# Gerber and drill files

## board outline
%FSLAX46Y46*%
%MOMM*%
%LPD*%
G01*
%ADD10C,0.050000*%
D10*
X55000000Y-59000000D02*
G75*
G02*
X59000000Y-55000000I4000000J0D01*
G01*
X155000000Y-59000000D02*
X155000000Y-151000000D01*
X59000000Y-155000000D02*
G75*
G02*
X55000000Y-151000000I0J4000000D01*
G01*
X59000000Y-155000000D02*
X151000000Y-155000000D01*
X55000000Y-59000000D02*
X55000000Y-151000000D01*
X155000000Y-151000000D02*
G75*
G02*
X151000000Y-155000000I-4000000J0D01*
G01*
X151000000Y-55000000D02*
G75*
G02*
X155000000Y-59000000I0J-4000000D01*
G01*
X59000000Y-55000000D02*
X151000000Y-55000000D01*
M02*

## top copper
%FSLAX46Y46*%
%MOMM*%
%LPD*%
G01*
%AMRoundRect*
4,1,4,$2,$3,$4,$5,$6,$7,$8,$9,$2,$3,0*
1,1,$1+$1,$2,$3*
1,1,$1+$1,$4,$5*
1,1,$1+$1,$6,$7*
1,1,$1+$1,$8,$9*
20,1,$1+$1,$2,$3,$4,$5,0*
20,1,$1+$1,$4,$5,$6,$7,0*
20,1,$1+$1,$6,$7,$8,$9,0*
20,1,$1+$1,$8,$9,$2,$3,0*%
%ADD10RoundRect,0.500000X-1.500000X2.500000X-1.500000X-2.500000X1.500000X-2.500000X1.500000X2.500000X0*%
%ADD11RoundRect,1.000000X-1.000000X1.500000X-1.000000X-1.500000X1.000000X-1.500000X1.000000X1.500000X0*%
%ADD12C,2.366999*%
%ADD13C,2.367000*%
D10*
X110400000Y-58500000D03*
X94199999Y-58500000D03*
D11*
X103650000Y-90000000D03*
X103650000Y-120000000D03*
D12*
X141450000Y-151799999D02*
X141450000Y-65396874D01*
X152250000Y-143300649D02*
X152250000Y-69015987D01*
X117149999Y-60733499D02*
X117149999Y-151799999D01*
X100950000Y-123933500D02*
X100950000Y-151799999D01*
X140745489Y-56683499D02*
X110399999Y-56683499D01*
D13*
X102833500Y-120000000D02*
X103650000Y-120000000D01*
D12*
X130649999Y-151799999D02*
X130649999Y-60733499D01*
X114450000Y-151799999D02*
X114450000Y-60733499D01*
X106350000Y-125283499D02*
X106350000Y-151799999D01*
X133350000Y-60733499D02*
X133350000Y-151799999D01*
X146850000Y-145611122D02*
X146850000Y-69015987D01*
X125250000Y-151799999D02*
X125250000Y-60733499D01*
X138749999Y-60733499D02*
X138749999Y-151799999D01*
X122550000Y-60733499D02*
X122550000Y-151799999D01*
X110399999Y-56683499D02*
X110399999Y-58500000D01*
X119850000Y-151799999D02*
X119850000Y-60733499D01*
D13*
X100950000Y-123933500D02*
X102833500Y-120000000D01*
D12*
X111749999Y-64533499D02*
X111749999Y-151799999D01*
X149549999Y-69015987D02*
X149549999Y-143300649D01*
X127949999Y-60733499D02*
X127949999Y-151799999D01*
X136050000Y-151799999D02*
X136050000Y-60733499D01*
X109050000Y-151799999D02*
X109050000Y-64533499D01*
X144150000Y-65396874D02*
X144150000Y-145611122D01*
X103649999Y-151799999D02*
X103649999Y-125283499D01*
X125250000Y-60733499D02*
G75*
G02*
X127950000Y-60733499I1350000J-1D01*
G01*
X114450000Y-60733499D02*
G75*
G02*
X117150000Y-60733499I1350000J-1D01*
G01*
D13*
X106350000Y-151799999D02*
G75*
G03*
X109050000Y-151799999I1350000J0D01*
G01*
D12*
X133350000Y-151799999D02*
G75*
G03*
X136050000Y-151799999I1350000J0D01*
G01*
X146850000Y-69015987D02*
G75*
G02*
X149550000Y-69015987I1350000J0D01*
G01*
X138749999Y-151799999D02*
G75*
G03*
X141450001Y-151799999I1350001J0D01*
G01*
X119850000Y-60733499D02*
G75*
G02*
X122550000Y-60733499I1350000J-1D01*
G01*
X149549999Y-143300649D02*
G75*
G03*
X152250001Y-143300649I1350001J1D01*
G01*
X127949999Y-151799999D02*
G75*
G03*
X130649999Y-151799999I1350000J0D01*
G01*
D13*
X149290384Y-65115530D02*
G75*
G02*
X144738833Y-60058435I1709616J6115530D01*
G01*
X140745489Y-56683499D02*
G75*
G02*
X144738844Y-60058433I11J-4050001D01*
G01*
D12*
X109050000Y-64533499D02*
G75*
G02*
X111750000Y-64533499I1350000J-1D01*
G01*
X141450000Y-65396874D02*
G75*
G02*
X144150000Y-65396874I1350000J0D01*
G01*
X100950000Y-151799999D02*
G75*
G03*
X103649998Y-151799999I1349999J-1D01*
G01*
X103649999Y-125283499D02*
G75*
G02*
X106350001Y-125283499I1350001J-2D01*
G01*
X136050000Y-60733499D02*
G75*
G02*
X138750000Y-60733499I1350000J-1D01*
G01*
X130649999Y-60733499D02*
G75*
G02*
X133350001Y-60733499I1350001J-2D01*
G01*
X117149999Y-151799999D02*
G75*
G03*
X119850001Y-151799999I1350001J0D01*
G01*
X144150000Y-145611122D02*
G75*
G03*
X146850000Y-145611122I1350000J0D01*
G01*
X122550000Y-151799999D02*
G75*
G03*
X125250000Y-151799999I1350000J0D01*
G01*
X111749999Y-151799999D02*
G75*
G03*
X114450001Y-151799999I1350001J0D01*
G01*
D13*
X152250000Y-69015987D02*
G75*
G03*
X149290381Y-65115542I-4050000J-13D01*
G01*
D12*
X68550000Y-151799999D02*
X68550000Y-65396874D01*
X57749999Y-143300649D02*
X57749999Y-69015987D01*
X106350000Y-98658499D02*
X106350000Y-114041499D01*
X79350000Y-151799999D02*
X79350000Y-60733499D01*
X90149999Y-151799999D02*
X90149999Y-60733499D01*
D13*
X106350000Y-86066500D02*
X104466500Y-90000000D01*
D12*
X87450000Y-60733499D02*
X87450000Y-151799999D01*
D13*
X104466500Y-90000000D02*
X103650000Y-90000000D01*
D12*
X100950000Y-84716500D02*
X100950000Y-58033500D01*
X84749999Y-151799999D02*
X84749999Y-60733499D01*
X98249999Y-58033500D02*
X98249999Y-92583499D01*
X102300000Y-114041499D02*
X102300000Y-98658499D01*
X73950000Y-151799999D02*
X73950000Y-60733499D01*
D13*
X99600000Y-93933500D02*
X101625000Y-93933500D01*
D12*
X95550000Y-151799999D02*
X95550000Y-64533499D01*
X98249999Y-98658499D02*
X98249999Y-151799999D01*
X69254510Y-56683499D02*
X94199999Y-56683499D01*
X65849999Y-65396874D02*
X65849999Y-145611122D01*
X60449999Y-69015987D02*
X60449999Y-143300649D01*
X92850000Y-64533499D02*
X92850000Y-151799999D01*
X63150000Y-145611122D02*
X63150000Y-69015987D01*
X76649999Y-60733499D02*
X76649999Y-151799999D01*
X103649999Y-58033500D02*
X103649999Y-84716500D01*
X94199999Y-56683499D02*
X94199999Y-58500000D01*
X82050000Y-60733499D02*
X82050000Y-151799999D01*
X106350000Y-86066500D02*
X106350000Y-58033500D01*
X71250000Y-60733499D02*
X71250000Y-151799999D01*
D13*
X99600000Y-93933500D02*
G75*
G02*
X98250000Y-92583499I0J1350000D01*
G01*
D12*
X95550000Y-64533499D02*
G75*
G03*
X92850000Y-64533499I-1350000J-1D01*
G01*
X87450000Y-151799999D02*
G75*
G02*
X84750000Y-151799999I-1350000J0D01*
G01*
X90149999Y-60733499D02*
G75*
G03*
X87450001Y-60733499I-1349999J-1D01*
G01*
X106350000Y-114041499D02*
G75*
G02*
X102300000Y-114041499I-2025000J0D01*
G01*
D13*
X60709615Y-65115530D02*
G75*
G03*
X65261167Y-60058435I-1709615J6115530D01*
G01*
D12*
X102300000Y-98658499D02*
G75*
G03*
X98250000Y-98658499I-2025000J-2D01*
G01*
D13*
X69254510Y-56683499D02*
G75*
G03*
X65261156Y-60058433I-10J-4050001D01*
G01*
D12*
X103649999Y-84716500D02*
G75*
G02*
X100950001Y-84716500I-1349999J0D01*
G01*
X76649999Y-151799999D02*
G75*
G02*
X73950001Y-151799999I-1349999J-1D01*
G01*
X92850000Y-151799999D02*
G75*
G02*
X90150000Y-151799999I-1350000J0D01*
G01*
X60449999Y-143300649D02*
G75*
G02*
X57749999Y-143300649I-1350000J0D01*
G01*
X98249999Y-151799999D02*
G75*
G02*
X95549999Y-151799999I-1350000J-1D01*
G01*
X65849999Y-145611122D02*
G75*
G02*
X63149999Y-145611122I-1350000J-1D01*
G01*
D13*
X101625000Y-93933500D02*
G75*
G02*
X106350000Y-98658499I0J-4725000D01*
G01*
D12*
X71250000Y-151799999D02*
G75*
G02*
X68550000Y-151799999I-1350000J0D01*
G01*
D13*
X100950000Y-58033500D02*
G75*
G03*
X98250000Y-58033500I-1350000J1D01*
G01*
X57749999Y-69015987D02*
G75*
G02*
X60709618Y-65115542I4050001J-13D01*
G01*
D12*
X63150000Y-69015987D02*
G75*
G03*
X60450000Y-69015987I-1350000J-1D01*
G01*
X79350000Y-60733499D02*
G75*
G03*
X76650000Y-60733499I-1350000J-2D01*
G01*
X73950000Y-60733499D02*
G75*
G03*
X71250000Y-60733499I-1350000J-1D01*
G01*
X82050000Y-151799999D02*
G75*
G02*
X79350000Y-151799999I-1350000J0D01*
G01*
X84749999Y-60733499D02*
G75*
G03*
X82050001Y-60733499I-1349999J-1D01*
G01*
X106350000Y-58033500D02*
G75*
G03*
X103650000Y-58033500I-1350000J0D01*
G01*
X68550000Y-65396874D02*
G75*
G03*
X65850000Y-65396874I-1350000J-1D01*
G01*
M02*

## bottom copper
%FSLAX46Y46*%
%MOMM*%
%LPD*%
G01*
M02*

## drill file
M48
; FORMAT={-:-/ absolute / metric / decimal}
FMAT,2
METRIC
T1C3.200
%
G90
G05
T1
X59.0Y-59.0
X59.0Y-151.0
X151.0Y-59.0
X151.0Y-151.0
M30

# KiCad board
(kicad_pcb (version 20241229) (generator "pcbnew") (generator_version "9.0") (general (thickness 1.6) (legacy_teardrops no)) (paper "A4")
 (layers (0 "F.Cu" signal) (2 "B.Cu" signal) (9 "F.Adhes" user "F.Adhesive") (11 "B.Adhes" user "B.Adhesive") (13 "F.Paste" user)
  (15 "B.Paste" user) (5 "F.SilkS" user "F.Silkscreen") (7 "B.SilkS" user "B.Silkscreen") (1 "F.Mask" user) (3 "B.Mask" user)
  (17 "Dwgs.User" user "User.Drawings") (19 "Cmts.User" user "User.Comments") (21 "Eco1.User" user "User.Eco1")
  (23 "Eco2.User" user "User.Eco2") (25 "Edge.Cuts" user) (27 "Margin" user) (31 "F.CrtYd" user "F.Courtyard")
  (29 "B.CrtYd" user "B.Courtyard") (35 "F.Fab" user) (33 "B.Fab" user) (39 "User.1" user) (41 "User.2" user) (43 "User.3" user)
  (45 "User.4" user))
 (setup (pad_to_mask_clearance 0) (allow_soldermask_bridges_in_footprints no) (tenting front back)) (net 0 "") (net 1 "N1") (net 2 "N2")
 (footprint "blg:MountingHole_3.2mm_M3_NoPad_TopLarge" (layer "F.Cu") (at 151 59)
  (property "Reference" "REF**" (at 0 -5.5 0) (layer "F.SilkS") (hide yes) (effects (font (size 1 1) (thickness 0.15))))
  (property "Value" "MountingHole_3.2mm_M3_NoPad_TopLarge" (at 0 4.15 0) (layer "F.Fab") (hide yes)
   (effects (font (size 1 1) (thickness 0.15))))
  (pad "" np_thru_hole circle (at 0 0) (size 7.6 7.6) (drill 3.2) (layers) (zone_connect 2)))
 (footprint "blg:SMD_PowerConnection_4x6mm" (layer "F.Cu") (at 110.4 58.5 -90)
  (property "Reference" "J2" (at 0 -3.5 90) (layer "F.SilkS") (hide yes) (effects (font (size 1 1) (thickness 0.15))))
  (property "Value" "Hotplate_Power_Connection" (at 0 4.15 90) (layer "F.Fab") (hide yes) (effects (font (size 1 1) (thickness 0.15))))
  (pad "1" smd roundrect (at 0 0 270) (size 6 4) (layers "F.Cu" "F.Mask" "F.Paste") (roundrect_rratio 0.125) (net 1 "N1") (zone_connect 2)))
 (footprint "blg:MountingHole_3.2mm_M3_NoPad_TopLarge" (layer "F.Cu") (at 59 151)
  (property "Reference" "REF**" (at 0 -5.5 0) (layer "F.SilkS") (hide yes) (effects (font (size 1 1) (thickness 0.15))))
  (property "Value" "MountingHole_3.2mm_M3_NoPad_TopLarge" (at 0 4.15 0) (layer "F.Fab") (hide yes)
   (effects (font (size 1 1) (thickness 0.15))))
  (pad "" np_thru_hole circle (at 0 0) (size 7.6 7.6) (drill 3.2) (layers) (zone_connect 2)))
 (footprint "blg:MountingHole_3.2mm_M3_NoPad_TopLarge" (layer "F.Cu") (at 151 151)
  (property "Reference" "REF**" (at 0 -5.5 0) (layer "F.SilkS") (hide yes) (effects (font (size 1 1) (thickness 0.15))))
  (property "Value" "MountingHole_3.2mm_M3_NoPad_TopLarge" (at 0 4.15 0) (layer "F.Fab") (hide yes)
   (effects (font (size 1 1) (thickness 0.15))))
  (pad "" np_thru_hole circle (at 0 0) (size 7.6 7.6) (drill 3.2) (layers) (zone_connect 2)))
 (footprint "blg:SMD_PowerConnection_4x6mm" (layer "F.Cu") (at 94.199999 58.5 -90)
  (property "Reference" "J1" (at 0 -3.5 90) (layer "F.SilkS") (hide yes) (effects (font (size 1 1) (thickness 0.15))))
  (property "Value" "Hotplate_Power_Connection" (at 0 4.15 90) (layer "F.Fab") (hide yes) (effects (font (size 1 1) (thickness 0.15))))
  (pad "1" smd roundrect (at 0 0 270) (size 6 4) (layers "F.Cu" "F.Mask" "F.Paste") (roundrect_rratio 0.125) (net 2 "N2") (zone_connect 2)))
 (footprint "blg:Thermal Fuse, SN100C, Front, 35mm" (layer "F.Cu") (at 103.65 105 -90)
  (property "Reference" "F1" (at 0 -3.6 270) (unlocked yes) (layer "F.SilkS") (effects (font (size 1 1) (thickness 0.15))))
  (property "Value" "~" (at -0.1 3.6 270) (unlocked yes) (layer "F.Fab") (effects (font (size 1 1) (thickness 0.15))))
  (pad "1" smd roundrect (at -15 0 270) (size 5 4) (layers "F.Cu" "F.Mask") (roundrect_rratio 0.25) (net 2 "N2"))
  (pad "2" smd roundrect (at 15 0 270) (size 5 4) (layers "F.Cu" "F.Mask") (roundrect_rratio 0.25) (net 1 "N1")))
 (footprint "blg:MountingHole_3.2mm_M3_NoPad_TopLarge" (layer "F.Cu") (at 59 59)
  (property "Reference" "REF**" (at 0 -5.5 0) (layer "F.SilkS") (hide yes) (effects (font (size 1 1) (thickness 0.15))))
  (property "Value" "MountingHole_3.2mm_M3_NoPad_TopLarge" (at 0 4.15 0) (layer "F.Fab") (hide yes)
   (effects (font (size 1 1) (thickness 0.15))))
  (pad "" np_thru_hole circle (at 0 0) (size 7.6 7.6) (drill 3.2) (layers) (zone_connect 2)))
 (gr_arc (start 55 59) (mid 56.171573 56.171573) (end 59 55) (stroke (width 0.05) (type solid)) (layer "Edge.Cuts"))
 (gr_line (start 155 59) (end 155 151) (stroke (width 0.05) (type default)) (layer "Edge.Cuts"))
 (gr_arc (start 59 155) (mid 56.171573 153.828427) (end 55 151) (stroke (width 0.05) (type solid)) (layer "Edge.Cuts"))
 (gr_line (start 59 155) (end 151 155) (stroke (width 0.05) (type default)) (layer "Edge.Cuts"))
 (gr_line (start 55 59) (end 55 151) (stroke (width 0.05) (type default)) (layer "Edge.Cuts"))
 (gr_arc (start 155 151) (mid 153.828427 153.828427) (end 151 155) (stroke (width 0.05) (type solid)) (layer "Edge.Cuts"))
 (gr_arc (start 151 55) (mid 153.828427 56.171573) (end 155 59) (stroke (width 0.05) (type solid)) (layer "Edge.Cuts"))
 (gr_line (start 59 55) (end 151 55) (stroke (width 0.05) (type default)) (layer "Edge.Cuts"))
 (segment (start 141.45 151.799999) (end 141.45 65.396874) (width 2.366999) (layer "F.Cu") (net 1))
 (segment (start 152.25 143.300649) (end 152.25 69.015987) (width 2.366999) (layer "F.Cu") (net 1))
 (segment (start 117.149999 60.733499) (end 117.149999 151.799999) (width 2.366999) (layer "F.Cu") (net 1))
 (segment (start 100.95 123.9335) (end 100.95 151.799999) (width 2.366999) (layer "F.Cu") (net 1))
 (segment (start 140.745489 56.683499) (end 110.399999 56.683499) (width 2.366999) (layer "F.Cu") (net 1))
 (segment (start 102.8335 120) (end 103.65 120) (width 2.367) (layer "F.Cu") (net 1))
 (segment (start 130.649999 151.799999) (end 130.649999 60.733499) (width 2.366999) (layer "F.Cu") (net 1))
 (segment (start 114.45 151.799999) (end 114.45 60.733499) (width 2.366999) (layer "F.Cu") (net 1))
 (segment (start 106.35 125.283499) (end 106.35 151.799999) (width 2.366999) (layer "F.Cu") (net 1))
 (segment (start 133.35 60.733499) (end 133.35 151.799999) (width 2.366999) (layer "F.Cu") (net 1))
 (segment (start 146.85 145.611122) (end 146.85 69.015987) (width 2.366999) (layer "F.Cu") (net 1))
 (segment (start 125.25 151.799999) (end 125.25 60.733499) (width 2.366999) (layer "F.Cu") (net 1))
 (segment (start 138.749999 60.733499) (end 138.749999 151.799999) (width 2.366999) (layer "F.Cu") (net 1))
 (segment (start 122.55 60.733499) (end 122.55 151.799999) (width 2.366999) (layer "F.Cu") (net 1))
 (segment (start 110.399999 56.683499) (end 110.399999 58.5) (width 2.366999) (layer "F.Cu") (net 1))
 (segment (start 119.85 151.799999) (end 119.85 60.733499) (width 2.366999) (layer "F.Cu") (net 1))
 (segment (start 100.95 123.9335) (end 102.8335 120) (width 2.367) (layer "F.Cu") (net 1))
 (segment (start 111.749999 64.533499) (end 111.749999 151.799999) (width 2.366999) (layer "F.Cu") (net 1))
 (segment (start 149.549999 69.015987) (end 149.549999 143.300649) (width 2.366999) (layer "F.Cu") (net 1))
 (segment (start 127.949999 60.733499) (end 127.949999 151.799999) (width 2.366999) (layer "F.Cu") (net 1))
 (segment (start 136.05 151.799999) (end 136.05 60.733499) (width 2.366999) (layer "F.Cu") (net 1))
 (segment (start 109.05 151.799999) (end 109.05 64.533499) (width 2.366999) (layer "F.Cu") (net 1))
 (segment (start 144.15 65.396874) (end 144.15 145.611122) (width 2.366999) (layer "F.Cu") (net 1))
 (segment (start 103.649999 151.799999) (end 103.649999 125.283499) (width 2.366999) (layer "F.Cu") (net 1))
 (arc (start 125.25 60.733499) (mid 126.6 59.3835) (end 127.949999 60.733499) (width 2.366999) (layer "F.Cu") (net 1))
 (arc (start 114.45 60.733499) (mid 115.8 59.3835) (end 117.149999 60.733499) (width 2.366999) (layer "F.Cu") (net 1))
 (arc (start 106.35 151.799999) (mid 107.7 153.149999) (end 109.05 151.799999) (width 2.367) (layer "F.Cu") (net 1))
 (arc (start 133.35 151.799999) (mid 134.7 153.149999) (end 136.05 151.799999) (width 2.366999) (layer "F.Cu") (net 1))
 (arc (start 146.85 69.015987) (mid 148.2 67.665987) (end 149.549999 69.015987) (width 2.366999) (layer "F.Cu") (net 1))
 (arc (start 138.749999 151.799999) (mid 140.1 153.149999) (end 141.45 151.799999) (width 2.366999) (layer "F.Cu") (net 1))
 (arc (start 119.85 60.733499) (mid 121.199999 59.3835) (end 122.55 60.733499) (width 2.366999) (layer "F.Cu") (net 1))
 (arc (start 149.549999 143.300649) (mid 150.9 144.650649) (end 152.25 143.300649) (width 2.366999) (layer "F.Cu") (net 1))
 (arc (start 127.949999 151.799999) (mid 129.3 153.149999) (end 130.649999 151.799999) (width 2.366999) (layer "F.Cu") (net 1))
 (arc (start 149.290384 65.11553) (mid 146.280159 63.248011) (end 144.738832 60.058435) (width 2.367) (layer "F.Cu") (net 1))
 (arc (start 140.745489 56.683499) (mid 143.359728 57.64024) (end 144.738832 60.058435) (width 2.367) (layer "F.Cu") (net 1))
 (arc (start 109.05 64.533499) (mid 110.399999 63.1835) (end 111.749999 64.533499) (width 2.366999) (layer "F.Cu") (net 1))
 (arc (start 141.45 65.396874) (mid 142.799999 64.046874) (end 144.15 65.396874) (width 2.366999) (layer "F.Cu") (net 1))
 (arc (start 100.95 151.799999) (mid 102.3 153.149999) (end 103.649999 151.799999) (width 2.366999) (layer "F.Cu") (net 1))
 (arc (start 103.649999 125.283499) (mid 105 123.9335) (end 106.35 125.283499) (width 2.366999) (layer "F.Cu") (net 1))
 (arc (start 136.05 60.733499) (mid 137.4 59.3835) (end 138.749999 60.733499) (width 2.366999) (layer "F.Cu") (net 1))
 (arc (start 130.649999 60.733499) (mid 132 59.3835) (end 133.35 60.733499) (width 2.366999) (layer "F.Cu") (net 1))
 (arc (start 117.149999 151.799999) (mid 118.5 153.149999) (end 119.85 151.799999) (width 2.366999) (layer "F.Cu") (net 1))
 (arc (start 144.15 145.611122) (mid 145.5 146.961122) (end 146.85 145.611122) (width 2.366999) (layer "F.Cu") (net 1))
 (arc (start 122.55 151.799999) (mid 123.899999 153.149999) (end 125.25 151.799999) (width 2.366999) (layer "F.Cu") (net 1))
 (arc (start 111.749999 151.799999) (mid 113.1 153.149999) (end 114.45 151.799999) (width 2.366999) (layer "F.Cu") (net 1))
 (arc (start 152.25 69.015987) (mid 151.04468 66.133229) (end 149.290384 65.11553) (width 2.367) (layer "F.Cu") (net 1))
 (segment (start 68.55 151.799999) (end 68.55 65.396874) (width 2.366999) (layer "F.Cu") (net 2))
 (segment (start 57.749999 143.300649) (end 57.749999 69.015987) (width 2.366999) (layer "F.Cu") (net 2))
 (segment (start 106.35 98.658499) (end 106.35 114.041499) (width 2.366999) (layer "F.Cu") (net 2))
 (segment (start 79.35 151.799999) (end 79.35 60.733499) (width 2.366999) (layer "F.Cu") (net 2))
 (segment (start 90.149999 151.799999) (end 90.149999 60.733499) (width 2.366999) (layer "F.Cu") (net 2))
 (segment (start 106.35 86.0665) (end 104.4665 90) (width 2.367) (layer "F.Cu") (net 2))
 (segment (start 87.45 60.733499) (end 87.45 151.799999) (width 2.366999) (layer "F.Cu") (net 2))
 (segment (start 104.4665 90) (end 103.65 90) (width 2.367) (layer "F.Cu") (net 2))
 (segment (start 100.95 84.7165) (end 100.95 58.0335) (width 2.366999) (layer "F.Cu") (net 2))
 (segment (start 84.749999 151.799999) (end 84.749999 60.733499) (width 2.366999) (layer "F.Cu") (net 2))
 (segment (start 98.249999 58.0335) (end 98.249999 92.583499) (width 2.366999) (layer "F.Cu") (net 2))
 (segment (start 102.3 114.041499) (end 102.3 98.658499) (width 2.366999) (layer "F.Cu") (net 2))
 (segment (start 73.95 151.799999) (end 73.95 60.733499) (width 2.366999) (layer "F.Cu") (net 2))
 (segment (start 99.6 93.9335) (end 101.625 93.9335) (width 2.367) (layer "F.Cu") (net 2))
 (segment (start 95.55 151.799999) (end 95.55 64.533499) (width 2.366999) (layer "F.Cu") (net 2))
 (segment (start 98.249999 98.658499) (end 98.249999 151.799999) (width 2.366999) (layer "F.Cu") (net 2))
 (segment (start 69.25451 56.683499) (end 94.199999 56.683499) (width 2.366999) (layer "F.Cu") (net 2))
 (segment (start 65.849999 65.396874) (end 65.849999 145.611122) (width 2.366999) (layer "F.Cu") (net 2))
 (segment (start 60.449999 69.015987) (end 60.449999 143.300649) (width 2.366999) (layer "F.Cu") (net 2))
 (segment (start 92.85 64.533499) (end 92.85 151.799999) (width 2.366999) (layer "F.Cu") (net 2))
 (segment (start 63.15 145.611122) (end 63.15 69.015987) (width 2.366999) (layer "F.Cu") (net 2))
 (segment (start 76.649999 60.733499) (end 76.649999 151.799999) (width 2.366999) (layer "F.Cu") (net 2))
 (segment (start 103.649999 58.0335) (end 103.649999 84.7165) (width 2.366999) (layer "F.Cu") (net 2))
 (segment (start 94.199999 56.683499) (end 94.199999 58.5) (width 2.366999) (layer "F.Cu") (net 2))
 (segment (start 82.05 60.733499) (end 82.05 151.799999) (width 2.366999) (layer "F.Cu") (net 2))
 (segment (start 106.35 86.0665) (end 106.35 58.0335) (width 2.366999) (layer "F.Cu") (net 2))
 (segment (start 71.25 60.733499) (end 71.25 151.799999) (width 2.366999) (layer "F.Cu") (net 2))
 (arc (start 99.6 93.9335) (mid 98.645405 93.538094) (end 98.249999 92.583499) (width 2.367) (layer "F.Cu") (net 2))
 (arc (start 95.55 64.533499) (mid 94.199999 63.1835) (end 92.85 64.533499) (width 2.366999) (layer "F.Cu") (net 2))
 (arc (start 87.45 151.799999) (mid 86.1 153.149999) (end 84.749999 151.799999) (width 2.366999) (layer "F.Cu") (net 2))
 (arc (start 90.149999 60.733499) (mid 88.799999 59.3835) (end 87.45 60.733499) (width 2.366999) (layer "F.Cu") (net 2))
 (arc (start 106.35 114.041499) (mid 104.325 116.066499) (end 102.3 114.041499) (width 2.366999) (layer "F.Cu") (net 2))
 (arc (start 60.709615 65.11553) (mid 63.71984 63.248011) (end 65.261167 60.058435) (width 2.367) (layer "F.Cu") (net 2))
 (arc (start 102.3 98.658499) (mid 100.274999 96.6335) (end 98.249999 98.658499) (width 2.366999) (layer "F.Cu") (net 2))
 (arc (start 69.25451 56.683499) (mid 66.640271 57.64024) (end 65.261167 60.058435) (width 2.367) (layer "F.Cu") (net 2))
 (arc (start 103.649999 84.7165) (mid 102.3 86.066499) (end 100.95 84.7165) (width 2.366999) (layer "F.Cu") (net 2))
 (arc (start 76.649999 151.799999) (mid 75.3 153.149999) (end 73.95 151.799999) (width 2.366999) (layer "F.Cu") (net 2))
 (arc (start 92.85 151.799999) (mid 91.5 153.149999) (end 90.149999 151.799999) (width 2.366999) (layer "F.Cu") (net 2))
 (arc (start 60.449999 143.300649) (mid 59.1 144.650649) (end 57.749999 143.300649) (width 2.366999) (layer "F.Cu") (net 2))
 (arc (start 98.249999 151.799999) (mid 96.9 153.149999) (end 95.55 151.799999) (width 2.366999) (layer "F.Cu") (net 2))
 (arc (start 65.849999 145.611122) (mid 64.5 146.961122) (end 63.15 145.611122) (width 2.366999) (layer "F.Cu") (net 2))
 (arc (start 101.625 93.9335) (mid 104.966079 95.31742) (end 106.35 98.658499) (width 2.367) (layer "F.Cu") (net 2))
 (arc (start 71.25 151.799999) (mid 69.899999 153.149999) (end 68.55 151.799999) (width 2.366999) (layer "F.Cu") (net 2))
 (arc (start 100.95 58.0335) (mid 99.6 56.683499) (end 98.25 58.0335) (width 2.367) (layer "F.Cu") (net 2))
 (arc (start 57.749999 69.015987) (mid 58.955319 66.133229) (end 60.709615 65.11553) (width 2.367) (layer "F.Cu") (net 2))
 (arc (start 63.15 69.015987) (mid 61.8 67.665987) (end 60.449999 69.015987) (width 2.366999) (layer "F.Cu") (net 2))
 (arc (start 79.35 60.733499) (mid 78 59.3835) (end 76.649999 60.733499) (width 2.366999) (layer "F.Cu") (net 2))
 (arc (start 73.95 60.733499) (mid 72.6 59.3835) (end 71.25 60.733499) (width 2.366999) (layer "F.Cu") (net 2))
 (arc (start 82.05 151.799999) (mid 80.699999 153.149999) (end 79.35 151.799999) (width 2.366999) (layer "F.Cu") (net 2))
 (arc (start 84.749999 60.733499) (mid 83.4 59.3835) (end 82.05 60.733499) (width 2.366999) (layer "F.Cu") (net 2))
 (arc (start 106.35 58.0335) (mid 105 56.683499) (end 103.649999 58.0335) (width 2.366999) (layer "F.Cu") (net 2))
 (arc (start 68.55 65.396874) (mid 67.2 64.046874) (end 65.849999 65.396874) (width 2.366999) (layer "F.Cu") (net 2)))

